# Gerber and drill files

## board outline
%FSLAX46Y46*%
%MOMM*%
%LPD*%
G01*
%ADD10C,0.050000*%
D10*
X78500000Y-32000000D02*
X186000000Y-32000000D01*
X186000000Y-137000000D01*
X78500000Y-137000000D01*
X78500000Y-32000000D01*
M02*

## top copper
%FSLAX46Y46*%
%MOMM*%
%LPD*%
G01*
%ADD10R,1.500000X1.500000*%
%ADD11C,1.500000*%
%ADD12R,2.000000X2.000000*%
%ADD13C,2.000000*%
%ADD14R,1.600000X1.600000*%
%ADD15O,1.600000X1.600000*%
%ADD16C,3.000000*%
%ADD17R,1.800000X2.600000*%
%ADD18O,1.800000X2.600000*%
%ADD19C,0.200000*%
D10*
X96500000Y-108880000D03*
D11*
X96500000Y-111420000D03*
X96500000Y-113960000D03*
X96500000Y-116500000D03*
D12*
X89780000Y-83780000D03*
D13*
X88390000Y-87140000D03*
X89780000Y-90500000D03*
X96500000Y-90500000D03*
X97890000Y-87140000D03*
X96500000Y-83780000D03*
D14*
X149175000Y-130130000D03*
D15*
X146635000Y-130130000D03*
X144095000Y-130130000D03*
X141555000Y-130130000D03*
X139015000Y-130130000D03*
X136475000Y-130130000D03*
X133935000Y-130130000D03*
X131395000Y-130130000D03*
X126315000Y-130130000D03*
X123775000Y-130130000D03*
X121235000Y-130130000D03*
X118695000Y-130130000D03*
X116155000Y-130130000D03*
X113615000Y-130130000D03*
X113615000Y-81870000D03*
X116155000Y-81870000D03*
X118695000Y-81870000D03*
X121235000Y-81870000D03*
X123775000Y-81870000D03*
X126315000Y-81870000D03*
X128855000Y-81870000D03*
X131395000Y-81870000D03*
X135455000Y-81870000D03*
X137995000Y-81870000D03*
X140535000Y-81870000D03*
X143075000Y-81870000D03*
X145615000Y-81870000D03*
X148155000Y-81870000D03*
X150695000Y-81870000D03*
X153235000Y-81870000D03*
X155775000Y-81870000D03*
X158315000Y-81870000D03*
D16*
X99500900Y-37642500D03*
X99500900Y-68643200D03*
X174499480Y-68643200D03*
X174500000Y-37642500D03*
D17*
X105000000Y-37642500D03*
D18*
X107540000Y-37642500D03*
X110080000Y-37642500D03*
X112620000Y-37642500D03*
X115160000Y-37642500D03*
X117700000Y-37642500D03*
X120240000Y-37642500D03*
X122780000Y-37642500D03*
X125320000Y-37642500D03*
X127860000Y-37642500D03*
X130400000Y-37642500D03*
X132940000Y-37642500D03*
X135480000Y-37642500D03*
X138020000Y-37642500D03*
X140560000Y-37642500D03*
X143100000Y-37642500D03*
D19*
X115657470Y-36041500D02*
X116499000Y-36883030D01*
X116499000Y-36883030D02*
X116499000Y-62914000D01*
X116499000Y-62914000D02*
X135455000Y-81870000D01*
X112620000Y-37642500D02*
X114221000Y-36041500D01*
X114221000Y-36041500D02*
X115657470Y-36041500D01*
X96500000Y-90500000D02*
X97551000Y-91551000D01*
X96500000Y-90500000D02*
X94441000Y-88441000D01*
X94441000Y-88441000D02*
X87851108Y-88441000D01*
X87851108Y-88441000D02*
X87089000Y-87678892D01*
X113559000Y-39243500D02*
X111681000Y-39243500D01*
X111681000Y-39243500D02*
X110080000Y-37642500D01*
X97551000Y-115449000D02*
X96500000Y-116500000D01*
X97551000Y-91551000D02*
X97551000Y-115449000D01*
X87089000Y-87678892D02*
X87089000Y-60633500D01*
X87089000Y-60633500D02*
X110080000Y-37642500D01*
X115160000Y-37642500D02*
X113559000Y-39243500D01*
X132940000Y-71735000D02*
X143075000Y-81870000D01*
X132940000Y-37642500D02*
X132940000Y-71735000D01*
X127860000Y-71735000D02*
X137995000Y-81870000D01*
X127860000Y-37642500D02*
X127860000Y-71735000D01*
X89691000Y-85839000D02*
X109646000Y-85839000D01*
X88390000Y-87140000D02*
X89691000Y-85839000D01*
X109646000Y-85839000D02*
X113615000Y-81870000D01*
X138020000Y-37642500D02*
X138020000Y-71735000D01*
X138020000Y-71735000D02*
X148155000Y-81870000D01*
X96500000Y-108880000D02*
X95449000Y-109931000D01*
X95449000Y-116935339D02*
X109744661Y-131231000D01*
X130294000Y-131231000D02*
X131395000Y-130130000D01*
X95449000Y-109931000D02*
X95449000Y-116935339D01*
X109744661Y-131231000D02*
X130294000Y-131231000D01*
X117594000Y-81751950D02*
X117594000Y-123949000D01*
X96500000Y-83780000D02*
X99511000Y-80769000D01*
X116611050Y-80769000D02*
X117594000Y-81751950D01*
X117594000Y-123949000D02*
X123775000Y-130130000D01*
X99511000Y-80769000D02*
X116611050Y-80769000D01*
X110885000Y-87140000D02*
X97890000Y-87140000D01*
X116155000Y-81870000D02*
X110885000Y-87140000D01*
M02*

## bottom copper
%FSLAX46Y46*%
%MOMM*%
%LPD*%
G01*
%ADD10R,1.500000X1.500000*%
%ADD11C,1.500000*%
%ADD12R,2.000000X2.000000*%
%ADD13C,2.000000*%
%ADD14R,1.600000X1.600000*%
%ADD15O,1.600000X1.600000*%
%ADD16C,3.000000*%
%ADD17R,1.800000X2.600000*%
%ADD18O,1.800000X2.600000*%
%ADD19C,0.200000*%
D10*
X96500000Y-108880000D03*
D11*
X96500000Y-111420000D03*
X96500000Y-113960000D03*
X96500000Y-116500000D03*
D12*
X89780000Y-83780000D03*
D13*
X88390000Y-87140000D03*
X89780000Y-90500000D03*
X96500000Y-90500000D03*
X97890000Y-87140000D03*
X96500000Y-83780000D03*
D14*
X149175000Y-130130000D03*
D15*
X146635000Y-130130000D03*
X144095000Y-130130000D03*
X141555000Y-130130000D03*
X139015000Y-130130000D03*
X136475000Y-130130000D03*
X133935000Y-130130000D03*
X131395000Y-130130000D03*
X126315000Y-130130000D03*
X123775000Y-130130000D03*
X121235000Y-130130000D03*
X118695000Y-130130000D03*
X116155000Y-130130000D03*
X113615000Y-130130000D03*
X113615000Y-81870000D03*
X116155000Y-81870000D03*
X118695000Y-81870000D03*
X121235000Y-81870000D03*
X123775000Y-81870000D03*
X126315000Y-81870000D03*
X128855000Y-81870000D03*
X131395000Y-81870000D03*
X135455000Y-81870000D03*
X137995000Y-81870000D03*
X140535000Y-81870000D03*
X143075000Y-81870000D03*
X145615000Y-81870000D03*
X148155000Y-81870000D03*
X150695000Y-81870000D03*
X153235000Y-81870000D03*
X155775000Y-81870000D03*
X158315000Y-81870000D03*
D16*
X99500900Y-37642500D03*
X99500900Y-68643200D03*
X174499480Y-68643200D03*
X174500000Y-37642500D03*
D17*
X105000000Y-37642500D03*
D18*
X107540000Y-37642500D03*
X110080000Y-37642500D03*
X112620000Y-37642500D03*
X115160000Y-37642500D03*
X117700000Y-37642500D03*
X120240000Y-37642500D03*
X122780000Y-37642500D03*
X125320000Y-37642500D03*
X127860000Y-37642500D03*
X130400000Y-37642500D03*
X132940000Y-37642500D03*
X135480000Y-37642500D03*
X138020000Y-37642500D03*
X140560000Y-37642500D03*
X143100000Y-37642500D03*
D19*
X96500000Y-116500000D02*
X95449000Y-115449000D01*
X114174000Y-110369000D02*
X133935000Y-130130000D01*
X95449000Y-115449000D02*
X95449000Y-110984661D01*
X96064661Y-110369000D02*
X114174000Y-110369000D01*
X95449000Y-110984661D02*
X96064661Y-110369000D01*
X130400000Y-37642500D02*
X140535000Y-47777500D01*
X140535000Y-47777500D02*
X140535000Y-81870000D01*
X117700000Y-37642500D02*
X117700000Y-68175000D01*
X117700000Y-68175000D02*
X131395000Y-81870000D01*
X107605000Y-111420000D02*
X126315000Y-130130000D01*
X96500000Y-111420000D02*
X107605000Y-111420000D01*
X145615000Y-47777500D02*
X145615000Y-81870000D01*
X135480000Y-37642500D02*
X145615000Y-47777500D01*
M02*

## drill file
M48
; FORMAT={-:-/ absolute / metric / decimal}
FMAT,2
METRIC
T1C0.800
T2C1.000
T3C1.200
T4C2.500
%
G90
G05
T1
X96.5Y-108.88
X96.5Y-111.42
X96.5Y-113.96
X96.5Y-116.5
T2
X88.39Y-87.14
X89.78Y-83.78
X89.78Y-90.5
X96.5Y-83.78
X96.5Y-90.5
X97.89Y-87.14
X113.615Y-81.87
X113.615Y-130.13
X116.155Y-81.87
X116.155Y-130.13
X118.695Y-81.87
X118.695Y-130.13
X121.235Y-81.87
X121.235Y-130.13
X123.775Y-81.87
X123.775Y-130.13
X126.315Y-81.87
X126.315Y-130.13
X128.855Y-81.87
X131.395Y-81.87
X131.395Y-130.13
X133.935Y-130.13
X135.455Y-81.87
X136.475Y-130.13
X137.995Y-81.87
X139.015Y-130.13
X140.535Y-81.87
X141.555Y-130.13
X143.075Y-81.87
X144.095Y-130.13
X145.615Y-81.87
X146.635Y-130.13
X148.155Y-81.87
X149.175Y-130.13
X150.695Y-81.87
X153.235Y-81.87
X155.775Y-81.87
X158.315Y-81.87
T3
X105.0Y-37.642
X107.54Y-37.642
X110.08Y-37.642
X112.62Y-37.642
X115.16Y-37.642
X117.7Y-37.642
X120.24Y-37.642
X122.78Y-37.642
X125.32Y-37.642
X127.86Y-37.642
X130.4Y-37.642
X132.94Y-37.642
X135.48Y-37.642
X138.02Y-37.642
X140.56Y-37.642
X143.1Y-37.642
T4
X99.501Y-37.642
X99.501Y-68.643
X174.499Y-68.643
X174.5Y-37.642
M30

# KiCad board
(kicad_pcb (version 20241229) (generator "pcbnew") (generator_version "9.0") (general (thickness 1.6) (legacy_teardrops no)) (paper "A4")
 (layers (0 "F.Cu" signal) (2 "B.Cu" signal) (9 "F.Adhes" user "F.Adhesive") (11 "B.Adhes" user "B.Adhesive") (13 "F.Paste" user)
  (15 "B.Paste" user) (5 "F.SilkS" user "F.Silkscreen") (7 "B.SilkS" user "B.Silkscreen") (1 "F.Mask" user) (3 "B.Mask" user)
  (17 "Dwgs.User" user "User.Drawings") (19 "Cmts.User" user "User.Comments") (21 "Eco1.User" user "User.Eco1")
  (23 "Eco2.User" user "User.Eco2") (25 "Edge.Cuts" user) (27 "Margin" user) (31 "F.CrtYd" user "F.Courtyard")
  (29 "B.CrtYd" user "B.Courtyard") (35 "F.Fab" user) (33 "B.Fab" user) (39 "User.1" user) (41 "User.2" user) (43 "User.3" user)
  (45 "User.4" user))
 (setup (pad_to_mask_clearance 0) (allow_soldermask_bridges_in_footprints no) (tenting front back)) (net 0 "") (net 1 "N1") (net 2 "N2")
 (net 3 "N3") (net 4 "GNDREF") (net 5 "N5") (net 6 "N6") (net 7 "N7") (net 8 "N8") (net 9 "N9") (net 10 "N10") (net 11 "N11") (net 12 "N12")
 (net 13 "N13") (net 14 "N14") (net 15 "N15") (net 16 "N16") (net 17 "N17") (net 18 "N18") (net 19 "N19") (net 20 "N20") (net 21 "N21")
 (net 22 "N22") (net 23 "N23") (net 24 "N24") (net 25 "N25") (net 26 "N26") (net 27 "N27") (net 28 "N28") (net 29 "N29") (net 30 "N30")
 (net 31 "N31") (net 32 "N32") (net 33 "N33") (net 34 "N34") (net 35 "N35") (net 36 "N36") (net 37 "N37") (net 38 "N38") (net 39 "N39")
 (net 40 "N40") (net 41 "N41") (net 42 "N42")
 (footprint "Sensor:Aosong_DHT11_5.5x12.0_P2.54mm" (layer "F.Cu") (at 96.5 108.88)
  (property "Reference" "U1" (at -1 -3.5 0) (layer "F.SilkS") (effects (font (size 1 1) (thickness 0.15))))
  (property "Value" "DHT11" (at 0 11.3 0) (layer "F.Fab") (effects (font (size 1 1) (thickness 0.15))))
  (pad "1" thru_hole rect (at 0 0) (size 1.5 1.5) (drill 0.8) (layers "*.Cu" "*.Mask") (remove_unused_layers no) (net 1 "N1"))
  (pad "2" thru_hole circle (at 0 2.54) (size 1.5 1.5) (drill 0.8) (layers "*.Cu" "*.Mask") (remove_unused_layers no) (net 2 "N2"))
  (pad "3" thru_hole circle (at 0 5.08) (size 1.5 1.5) (drill 0.8) (layers "*.Cu" "*.Mask") (remove_unused_layers no) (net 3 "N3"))
  (pad "4" thru_hole circle (at 0 7.62) (size 1.5 1.5) (drill 0.8) (layers "*.Cu" "*.Mask") (remove_unused_layers no) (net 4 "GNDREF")))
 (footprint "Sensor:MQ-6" (layer "F.Cu") (at 89.78 83.78)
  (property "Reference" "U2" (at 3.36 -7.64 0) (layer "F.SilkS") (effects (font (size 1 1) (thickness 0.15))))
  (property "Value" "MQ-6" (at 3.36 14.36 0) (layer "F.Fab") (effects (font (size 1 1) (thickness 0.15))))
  (pad "1" thru_hole rect (at 0 0) (size 2 2) (drill 1) (layers "*.Cu" "*.Mask") (remove_unused_layers no) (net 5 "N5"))
  (pad "2" thru_hole circle (at -1.39 3.36) (size 2 2) (drill 1) (layers "*.Cu" "*.Mask") (remove_unused_layers no) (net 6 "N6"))
  (pad "3" thru_hole circle (at 0 6.72 90) (size 2 2) (drill 1) (layers "*.Cu" "*.Mask") (remove_unused_layers no) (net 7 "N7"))
  (pad "4" thru_hole circle (at 6.72 6.72 180) (size 2 2) (drill 1) (layers "*.Cu" "*.Mask") (remove_unused_layers no) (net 4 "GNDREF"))
  (pad "5" thru_hole circle (at 8.11 3.36) (size 2 2) (drill 1) (layers "*.Cu" "*.Mask") (remove_unused_layers no) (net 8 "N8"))
  (pad "6" thru_hole circle (at 6.72 0 270) (size 2 2) (drill 1) (layers "*.Cu" "*.Mask") (remove_unused_layers no) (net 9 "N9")))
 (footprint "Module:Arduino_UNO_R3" (layer "F.Cu") (at 149.175 130.13 180)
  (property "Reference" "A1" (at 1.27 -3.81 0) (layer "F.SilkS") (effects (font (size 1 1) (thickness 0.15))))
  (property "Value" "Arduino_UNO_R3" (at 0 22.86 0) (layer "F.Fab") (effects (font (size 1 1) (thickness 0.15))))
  (pad "1" thru_hole rect (at 0 0 270) (size 1.6 1.6) (drill 1) (layers "*.Cu" "*.Mask") (remove_unused_layers no) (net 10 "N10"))
  (pad "2" thru_hole oval (at 2.54 0 270) (size 1.6 1.6) (drill 1) (layers "*.Cu" "*.Mask") (remove_unused_layers no) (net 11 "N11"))
  (pad "3" thru_hole oval (at 5.08 0 270) (size 1.6 1.6) (drill 1) (layers "*.Cu" "*.Mask") (remove_unused_layers no) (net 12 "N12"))
  (pad "4" thru_hole oval (at 7.62 0 270) (size 1.6 1.6) (drill 1) (layers "*.Cu" "*.Mask") (remove_unused_layers no) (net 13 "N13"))
  (pad "5" thru_hole oval (at 10.16 0 270) (size 1.6 1.6) (drill 1) (layers "*.Cu" "*.Mask") (remove_unused_layers no) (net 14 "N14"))
  (pad "6" thru_hole oval (at 12.7 0 270) (size 1.6 1.6) (drill 1) (layers "*.Cu" "*.Mask") (remove_unused_layers no) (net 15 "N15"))
  (pad "7" thru_hole oval (at 15.24 0 270) (size 1.6 1.6) (drill 1) (layers "*.Cu" "*.Mask") (remove_unused_layers no) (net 4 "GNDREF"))
  (pad "8" thru_hole oval (at 17.78 0 270) (size 1.6 1.6) (drill 1) (layers "*.Cu" "*.Mask") (remove_unused_layers no) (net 1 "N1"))
  (pad "9" thru_hole oval (at 22.86 0 270) (size 1.6 1.6) (drill 1) (layers "*.Cu" "*.Mask") (remove_unused_layers no) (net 2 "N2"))
  (pad "10" thru_hole oval (at 25.4 0 270) (size 1.6 1.6) (drill 1) (layers "*.Cu" "*.Mask") (remove_unused_layers no) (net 9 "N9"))
  (pad "11" thru_hole oval (at 27.94 0 270) (size 1.6 1.6) (drill 1) (layers "*.Cu" "*.Mask") (remove_unused_layers no) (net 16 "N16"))
  (pad "12" thru_hole oval (at 30.48 0 270) (size 1.6 1.6) (drill 1) (layers "*.Cu" "*.Mask") (remove_unused_layers no) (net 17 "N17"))
  (pad "13" thru_hole oval (at 33.02 0 270) (size 1.6 1.6) (drill 1) (layers "*.Cu" "*.Mask") (remove_unused_layers no) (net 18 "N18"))
  (pad "14" thru_hole oval (at 35.56 0 270) (size 1.6 1.6) (drill 1) (layers "*.Cu" "*.Mask") (remove_unused_layers no) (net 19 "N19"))
  (pad "15" thru_hole oval (at 35.56 48.26 270) (size 1.6 1.6) (drill 1) (layers "*.Cu" "*.Mask") (remove_unused_layers no) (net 6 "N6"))
  (pad "16" thru_hole oval (at 33.02 48.26 270) (size 1.6 1.6) (drill 1) (layers "*.Cu" "*.Mask") (remove_unused_layers no) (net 8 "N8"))
  (pad "17" thru_hole oval (at 30.48 48.26 270) (size 1.6 1.6) (drill 1) (layers "*.Cu" "*.Mask") (remove_unused_layers no) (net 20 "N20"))
  (pad "18" thru_hole oval (at 27.94 48.26 270) (size 1.6 1.6) (drill 1) (layers "*.Cu" "*.Mask") (remove_unused_layers no) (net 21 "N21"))
  (pad "19" thru_hole oval (at 25.4 48.26 270) (size 1.6 1.6) (drill 1) (layers "*.Cu" "*.Mask") (remove_unused_layers no) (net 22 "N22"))
  (pad "20" thru_hole oval (at 22.86 48.26 270) (size 1.6 1.6) (drill 1) (layers "*.Cu" "*.Mask") (remove_unused_layers no) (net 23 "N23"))
  (pad "21" thru_hole oval (at 20.32 48.26 270) (size 1.6 1.6) (drill 1) (layers "*.Cu" "*.Mask") (remove_unused_layers no) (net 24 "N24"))
  (pad "22" thru_hole oval (at 17.78 48.26 270) (size 1.6 1.6) (drill 1) (layers "*.Cu" "*.Mask") (remove_unused_layers no) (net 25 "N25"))
  (pad "23" thru_hole oval (at 13.72 48.26 270) (size 1.6 1.6) (drill 1) (layers "*.Cu" "*.Mask") (remove_unused_layers no) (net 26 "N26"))
  (pad "24" thru_hole oval (at 11.18 48.26 270) (size 1.6 1.6) (drill 1) (layers "*.Cu" "*.Mask") (remove_unused_layers no) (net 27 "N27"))
  (pad "25" thru_hole oval (at 8.64 48.26 270) (size 1.6 1.6) (drill 1) (layers "*.Cu" "*.Mask") (remove_unused_layers no) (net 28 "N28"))
  (pad "26" thru_hole oval (at 6.1 48.26 270) (size 1.6 1.6) (drill 1) (layers "*.Cu" "*.Mask") (remove_unused_layers no) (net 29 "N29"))
  (pad "27" thru_hole oval (at 3.56 48.26 270) (size 1.6 1.6) (drill 1) (layers "*.Cu" "*.Mask") (remove_unused_layers no) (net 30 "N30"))
  (pad "28" thru_hole oval (at 1.02 48.26 270) (size 1.6 1.6) (drill 1) (layers "*.Cu" "*.Mask") (remove_unused_layers no) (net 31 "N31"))
  (pad "29" thru_hole oval (at -1.52 48.26 270) (size 1.6 1.6) (drill 1) (layers "*.Cu" "*.Mask") (remove_unused_layers no) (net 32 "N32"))
  (pad "30" thru_hole oval (at -4.06 48.26 270) (size 1.6 1.6) (drill 1) (layers "*.Cu" "*.Mask") (remove_unused_layers no) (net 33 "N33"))
  (pad "31" thru_hole oval (at -6.6 48.26 270) (size 1.6 1.6) (drill 1) (layers "*.Cu" "*.Mask") (remove_unused_layers no) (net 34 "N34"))
  (pad "32" thru_hole oval (at -9.14 48.26 270) (size 1.6 1.6) (drill 1) (layers "*.Cu" "*.Mask") (remove_unused_layers no) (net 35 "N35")))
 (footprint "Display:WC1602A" (layer "F.Cu") (at 105 37.6425)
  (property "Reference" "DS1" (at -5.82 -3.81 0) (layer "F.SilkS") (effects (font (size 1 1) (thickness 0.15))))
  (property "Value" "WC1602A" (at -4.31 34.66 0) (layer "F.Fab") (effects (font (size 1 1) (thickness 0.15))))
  (pad "" thru_hole circle (at -5.4991 0) (size 3 3) (drill 2.5) (layers "*.Cu" "*.Mask") (remove_unused_layers no))
  (pad "" thru_hole circle (at -5.4991 31.0007) (size 3 3) (drill 2.5) (layers "*.Cu" "*.Mask") (remove_unused_layers no))
  (pad "" thru_hole circle (at 69.49948 31.0007) (size 3 3) (drill 2.5) (layers "*.Cu" "*.Mask") (remove_unused_layers no))
  (pad "" thru_hole circle (at 69.5 0) (size 3 3) (drill 2.5) (layers "*.Cu" "*.Mask") (remove_unused_layers no))
  (pad "1" thru_hole rect (at 0 0) (size 1.8 2.6) (drill 1.2) (layers "*.Cu" "*.Mask") (remove_unused_layers no) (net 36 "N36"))
  (pad "2" thru_hole oval (at 2.54 0) (size 1.8 2.6) (drill 1.2) (layers "*.Cu" "*.Mask") (remove_unused_layers no) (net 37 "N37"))
  (pad "3" thru_hole oval (at 5.08 0) (size 1.8 2.6) (drill 1.2) (layers "*.Cu" "*.Mask") (remove_unused_layers no) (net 4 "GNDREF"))
  (pad "4" thru_hole oval (at 7.62 0) (size 1.8 2.6) (drill 1.2) (layers "*.Cu" "*.Mask") (remove_unused_layers no) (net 26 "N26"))
  (pad "5" thru_hole oval (at 10.16 0) (size 1.8 2.6) (drill 1.2) (layers "*.Cu" "*.Mask") (remove_unused_layers no) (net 4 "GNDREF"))
  (pad "6" thru_hole oval (at 12.7 0) (size 1.8 2.6) (drill 1.2) (layers "*.Cu" "*.Mask") (remove_unused_layers no) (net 25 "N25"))
  (pad "7" thru_hole oval (at 15.24 0) (size 1.8 2.6) (drill 1.2) (layers "*.Cu" "*.Mask") (remove_unused_layers no) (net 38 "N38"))
  (pad "8" thru_hole oval (at 17.78 0) (size 1.8 2.6) (drill 1.2) (layers "*.Cu" "*.Mask") (remove_unused_layers no) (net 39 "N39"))
  (pad "9" thru_hole oval (at 20.32 0) (size 1.8 2.6) (drill 1.2) (layers "*.Cu" "*.Mask") (remove_unused_layers no) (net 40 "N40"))
  (pad "10" thru_hole oval (at 22.86 0) (size 1.8 2.6) (drill 1.2) (layers "*.Cu" "*.Mask") (remove_unused_layers no) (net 27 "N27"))
  (pad "11" thru_hole oval (at 25.4 0) (size 1.8 2.6) (drill 1.2) (layers "*.Cu" "*.Mask") (remove_unused_layers no) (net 28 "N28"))
  (pad "12" thru_hole oval (at 27.94 0) (size 1.8 2.6) (drill 1.2) (layers "*.Cu" "*.Mask") (remove_unused_layers no) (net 29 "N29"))
  (pad "13" thru_hole oval (at 30.48 0) (size 1.8 2.6) (drill 1.2) (layers "*.Cu" "*.Mask") (remove_unused_layers no) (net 30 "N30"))
  (pad "14" thru_hole oval (at 33.02 0) (size 1.8 2.6) (drill 1.2) (layers "*.Cu" "*.Mask") (remove_unused_layers no) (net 31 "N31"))
  (pad "15" thru_hole oval (at 35.56 0) (size 1.8 2.6) (drill 1.2) (layers "*.Cu" "*.Mask") (remove_unused_layers no) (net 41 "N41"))
  (pad "16" thru_hole oval (at 38.1 0) (size 1.8 2.6) (drill 1.2) (layers "*.Cu" "*.Mask") (remove_unused_layers no) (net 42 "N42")))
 (gr_rect (start 78.5 32) (end 186 137) (stroke (width 0.05) (type default)) (fill no) (layer "Edge.Cuts"))
 (segment (start 115.65747 36.0415) (end 116.499 36.88303) (width 0.2) (layer "F.Cu") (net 26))
 (segment (start 116.499 36.88303) (end 116.499 62.914) (width 0.2) (layer "F.Cu") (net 26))
 (segment (start 116.499 62.914) (end 135.455 81.87) (width 0.2) (layer "F.Cu") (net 26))
 (segment (start 112.62 37.6425) (end 114.221 36.0415) (width 0.2) (layer "F.Cu") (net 26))
 (segment (start 114.221 36.0415) (end 115.65747 36.0415) (width 0.2) (layer "F.Cu") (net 26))
 (segment (start 96.5 90.5) (end 97.551 91.551) (width 0.2) (layer "F.Cu") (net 4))
 (segment (start 96.5 90.5) (end 94.441 88.441) (width 0.2) (layer "F.Cu") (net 4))
 (segment (start 94.441 88.441) (end 87.851108 88.441) (width 0.2) (layer "F.Cu") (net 4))
 (segment (start 87.851108 88.441) (end 87.089 87.678892) (width 0.2) (layer "F.Cu") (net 4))
 (segment (start 113.559 39.2435) (end 111.681 39.2435) (width 0.2) (layer "F.Cu") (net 4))
 (segment (start 111.681 39.2435) (end 110.08 37.6425) (width 0.2) (layer "F.Cu") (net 4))
 (segment (start 97.551 115.449) (end 96.5 116.5) (width 0.2) (layer "F.Cu") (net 4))
 (segment (start 97.551 91.551) (end 97.551 115.449) (width 0.2) (layer "F.Cu") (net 4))
 (segment (start 87.089 87.678892) (end 87.089 60.6335) (width 0.2) (layer "F.Cu") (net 4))
 (segment (start 87.089 60.6335) (end 110.08 37.6425) (width 0.2) (layer "F.Cu") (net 4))
 (segment (start 115.16 37.6425) (end 113.559 39.2435) (width 0.2) (layer "F.Cu") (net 4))
 (segment (start 96.5 116.5) (end 95.449 115.449) (width 0.2) (layer "B.Cu") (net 4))
 (segment (start 114.174 110.369) (end 133.935 130.13) (width 0.2) (layer "B.Cu") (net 4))
 (segment (start 95.449 115.449) (end 95.449 110.984661) (width 0.2) (layer "B.Cu") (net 4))
 (segment (start 96.064661 110.369) (end 114.174 110.369) (width 0.2) (layer "B.Cu") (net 4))
 (segment (start 95.449 110.984661) (end 96.064661 110.369) (width 0.2) (layer "B.Cu") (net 4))
 (segment (start 130.4 37.6425) (end 140.535 47.7775) (width 0.2) (layer "B.Cu") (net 28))
 (segment (start 140.535 47.7775) (end 140.535 81.87) (width 0.2) (layer "B.Cu") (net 28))
 (segment (start 117.7 37.6425) (end 117.7 68.175) (width 0.2) (layer "B.Cu") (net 25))
 (segment (start 117.7 68.175) (end 131.395 81.87) (width 0.2) (layer "B.Cu") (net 25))
 (segment (start 132.94 71.735) (end 143.075 81.87) (width 0.2) (layer "F.Cu") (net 29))
 (segment (start 132.94 37.6425) (end 132.94 71.735) (width 0.2) (layer "F.Cu") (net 29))
 (segment (start 127.86 71.735) (end 137.995 81.87) (width 0.2) (layer "F.Cu") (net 27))
 (segment (start 127.86 37.6425) (end 127.86 71.735) (width 0.2) (layer "F.Cu") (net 27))
 (segment (start 89.691 85.839) (end 109.646 85.839) (width 0.2) (layer "F.Cu") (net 6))
 (segment (start 88.39 87.14) (end 89.691 85.839) (width 0.2) (layer "F.Cu") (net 6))
 (segment (start 109.646 85.839) (end 113.615 81.87) (width 0.2) (layer "F.Cu") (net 6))
 (segment (start 138.02 37.6425) (end 138.02 71.735) (width 0.2) (layer "F.Cu") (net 31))
 (segment (start 138.02 71.735) (end 148.155 81.87) (width 0.2) (layer "F.Cu") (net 31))
 (segment (start 96.5 108.88) (end 95.449 109.931) (width 0.2) (layer "F.Cu") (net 1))
 (segment (start 95.449 116.935339) (end 109.744661 131.231) (width 0.2) (layer "F.Cu") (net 1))
 (segment (start 130.294 131.231) (end 131.395 130.13) (width 0.2) (layer "F.Cu") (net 1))
 (segment (start 95.449 109.931) (end 95.449 116.935339) (width 0.2) (layer "F.Cu") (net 1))
 (segment (start 109.744661 131.231) (end 130.294 131.231) (width 0.2) (layer "F.Cu") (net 1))
 (segment (start 117.594 81.75195) (end 117.594 123.949) (width 0.2) (layer "F.Cu") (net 9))
 (segment (start 96.5 83.78) (end 99.511 80.769) (width 0.2) (layer "F.Cu") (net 9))
 (segment (start 116.61105 80.769) (end 117.594 81.75195) (width 0.2) (layer "F.Cu") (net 9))
 (segment (start 117.594 123.949) (end 123.775 130.13) (width 0.2) (layer "F.Cu") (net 9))
 (segment (start 99.511 80.769) (end 116.61105 80.769) (width 0.2) (layer "F.Cu") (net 9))
 (segment (start 107.605 111.42) (end 126.315 130.13) (width 0.2) (layer "B.Cu") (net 2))
 (segment (start 96.5 111.42) (end 107.605 111.42) (width 0.2) (layer "B.Cu") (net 2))
 (segment (start 145.615 47.7775) (end 145.615 81.87) (width 0.2) (layer "B.Cu") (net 30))
 (segment (start 135.48 37.6425) (end 145.615 47.7775) (width 0.2) (layer "B.Cu") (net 30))
 (segment (start 110.885 87.14) (end 97.89 87.14) (width 0.2) (layer "F.Cu") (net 8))
 (segment (start 116.155 81.87) (end 110.885 87.14) (width 0.2) (layer "F.Cu") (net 8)))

